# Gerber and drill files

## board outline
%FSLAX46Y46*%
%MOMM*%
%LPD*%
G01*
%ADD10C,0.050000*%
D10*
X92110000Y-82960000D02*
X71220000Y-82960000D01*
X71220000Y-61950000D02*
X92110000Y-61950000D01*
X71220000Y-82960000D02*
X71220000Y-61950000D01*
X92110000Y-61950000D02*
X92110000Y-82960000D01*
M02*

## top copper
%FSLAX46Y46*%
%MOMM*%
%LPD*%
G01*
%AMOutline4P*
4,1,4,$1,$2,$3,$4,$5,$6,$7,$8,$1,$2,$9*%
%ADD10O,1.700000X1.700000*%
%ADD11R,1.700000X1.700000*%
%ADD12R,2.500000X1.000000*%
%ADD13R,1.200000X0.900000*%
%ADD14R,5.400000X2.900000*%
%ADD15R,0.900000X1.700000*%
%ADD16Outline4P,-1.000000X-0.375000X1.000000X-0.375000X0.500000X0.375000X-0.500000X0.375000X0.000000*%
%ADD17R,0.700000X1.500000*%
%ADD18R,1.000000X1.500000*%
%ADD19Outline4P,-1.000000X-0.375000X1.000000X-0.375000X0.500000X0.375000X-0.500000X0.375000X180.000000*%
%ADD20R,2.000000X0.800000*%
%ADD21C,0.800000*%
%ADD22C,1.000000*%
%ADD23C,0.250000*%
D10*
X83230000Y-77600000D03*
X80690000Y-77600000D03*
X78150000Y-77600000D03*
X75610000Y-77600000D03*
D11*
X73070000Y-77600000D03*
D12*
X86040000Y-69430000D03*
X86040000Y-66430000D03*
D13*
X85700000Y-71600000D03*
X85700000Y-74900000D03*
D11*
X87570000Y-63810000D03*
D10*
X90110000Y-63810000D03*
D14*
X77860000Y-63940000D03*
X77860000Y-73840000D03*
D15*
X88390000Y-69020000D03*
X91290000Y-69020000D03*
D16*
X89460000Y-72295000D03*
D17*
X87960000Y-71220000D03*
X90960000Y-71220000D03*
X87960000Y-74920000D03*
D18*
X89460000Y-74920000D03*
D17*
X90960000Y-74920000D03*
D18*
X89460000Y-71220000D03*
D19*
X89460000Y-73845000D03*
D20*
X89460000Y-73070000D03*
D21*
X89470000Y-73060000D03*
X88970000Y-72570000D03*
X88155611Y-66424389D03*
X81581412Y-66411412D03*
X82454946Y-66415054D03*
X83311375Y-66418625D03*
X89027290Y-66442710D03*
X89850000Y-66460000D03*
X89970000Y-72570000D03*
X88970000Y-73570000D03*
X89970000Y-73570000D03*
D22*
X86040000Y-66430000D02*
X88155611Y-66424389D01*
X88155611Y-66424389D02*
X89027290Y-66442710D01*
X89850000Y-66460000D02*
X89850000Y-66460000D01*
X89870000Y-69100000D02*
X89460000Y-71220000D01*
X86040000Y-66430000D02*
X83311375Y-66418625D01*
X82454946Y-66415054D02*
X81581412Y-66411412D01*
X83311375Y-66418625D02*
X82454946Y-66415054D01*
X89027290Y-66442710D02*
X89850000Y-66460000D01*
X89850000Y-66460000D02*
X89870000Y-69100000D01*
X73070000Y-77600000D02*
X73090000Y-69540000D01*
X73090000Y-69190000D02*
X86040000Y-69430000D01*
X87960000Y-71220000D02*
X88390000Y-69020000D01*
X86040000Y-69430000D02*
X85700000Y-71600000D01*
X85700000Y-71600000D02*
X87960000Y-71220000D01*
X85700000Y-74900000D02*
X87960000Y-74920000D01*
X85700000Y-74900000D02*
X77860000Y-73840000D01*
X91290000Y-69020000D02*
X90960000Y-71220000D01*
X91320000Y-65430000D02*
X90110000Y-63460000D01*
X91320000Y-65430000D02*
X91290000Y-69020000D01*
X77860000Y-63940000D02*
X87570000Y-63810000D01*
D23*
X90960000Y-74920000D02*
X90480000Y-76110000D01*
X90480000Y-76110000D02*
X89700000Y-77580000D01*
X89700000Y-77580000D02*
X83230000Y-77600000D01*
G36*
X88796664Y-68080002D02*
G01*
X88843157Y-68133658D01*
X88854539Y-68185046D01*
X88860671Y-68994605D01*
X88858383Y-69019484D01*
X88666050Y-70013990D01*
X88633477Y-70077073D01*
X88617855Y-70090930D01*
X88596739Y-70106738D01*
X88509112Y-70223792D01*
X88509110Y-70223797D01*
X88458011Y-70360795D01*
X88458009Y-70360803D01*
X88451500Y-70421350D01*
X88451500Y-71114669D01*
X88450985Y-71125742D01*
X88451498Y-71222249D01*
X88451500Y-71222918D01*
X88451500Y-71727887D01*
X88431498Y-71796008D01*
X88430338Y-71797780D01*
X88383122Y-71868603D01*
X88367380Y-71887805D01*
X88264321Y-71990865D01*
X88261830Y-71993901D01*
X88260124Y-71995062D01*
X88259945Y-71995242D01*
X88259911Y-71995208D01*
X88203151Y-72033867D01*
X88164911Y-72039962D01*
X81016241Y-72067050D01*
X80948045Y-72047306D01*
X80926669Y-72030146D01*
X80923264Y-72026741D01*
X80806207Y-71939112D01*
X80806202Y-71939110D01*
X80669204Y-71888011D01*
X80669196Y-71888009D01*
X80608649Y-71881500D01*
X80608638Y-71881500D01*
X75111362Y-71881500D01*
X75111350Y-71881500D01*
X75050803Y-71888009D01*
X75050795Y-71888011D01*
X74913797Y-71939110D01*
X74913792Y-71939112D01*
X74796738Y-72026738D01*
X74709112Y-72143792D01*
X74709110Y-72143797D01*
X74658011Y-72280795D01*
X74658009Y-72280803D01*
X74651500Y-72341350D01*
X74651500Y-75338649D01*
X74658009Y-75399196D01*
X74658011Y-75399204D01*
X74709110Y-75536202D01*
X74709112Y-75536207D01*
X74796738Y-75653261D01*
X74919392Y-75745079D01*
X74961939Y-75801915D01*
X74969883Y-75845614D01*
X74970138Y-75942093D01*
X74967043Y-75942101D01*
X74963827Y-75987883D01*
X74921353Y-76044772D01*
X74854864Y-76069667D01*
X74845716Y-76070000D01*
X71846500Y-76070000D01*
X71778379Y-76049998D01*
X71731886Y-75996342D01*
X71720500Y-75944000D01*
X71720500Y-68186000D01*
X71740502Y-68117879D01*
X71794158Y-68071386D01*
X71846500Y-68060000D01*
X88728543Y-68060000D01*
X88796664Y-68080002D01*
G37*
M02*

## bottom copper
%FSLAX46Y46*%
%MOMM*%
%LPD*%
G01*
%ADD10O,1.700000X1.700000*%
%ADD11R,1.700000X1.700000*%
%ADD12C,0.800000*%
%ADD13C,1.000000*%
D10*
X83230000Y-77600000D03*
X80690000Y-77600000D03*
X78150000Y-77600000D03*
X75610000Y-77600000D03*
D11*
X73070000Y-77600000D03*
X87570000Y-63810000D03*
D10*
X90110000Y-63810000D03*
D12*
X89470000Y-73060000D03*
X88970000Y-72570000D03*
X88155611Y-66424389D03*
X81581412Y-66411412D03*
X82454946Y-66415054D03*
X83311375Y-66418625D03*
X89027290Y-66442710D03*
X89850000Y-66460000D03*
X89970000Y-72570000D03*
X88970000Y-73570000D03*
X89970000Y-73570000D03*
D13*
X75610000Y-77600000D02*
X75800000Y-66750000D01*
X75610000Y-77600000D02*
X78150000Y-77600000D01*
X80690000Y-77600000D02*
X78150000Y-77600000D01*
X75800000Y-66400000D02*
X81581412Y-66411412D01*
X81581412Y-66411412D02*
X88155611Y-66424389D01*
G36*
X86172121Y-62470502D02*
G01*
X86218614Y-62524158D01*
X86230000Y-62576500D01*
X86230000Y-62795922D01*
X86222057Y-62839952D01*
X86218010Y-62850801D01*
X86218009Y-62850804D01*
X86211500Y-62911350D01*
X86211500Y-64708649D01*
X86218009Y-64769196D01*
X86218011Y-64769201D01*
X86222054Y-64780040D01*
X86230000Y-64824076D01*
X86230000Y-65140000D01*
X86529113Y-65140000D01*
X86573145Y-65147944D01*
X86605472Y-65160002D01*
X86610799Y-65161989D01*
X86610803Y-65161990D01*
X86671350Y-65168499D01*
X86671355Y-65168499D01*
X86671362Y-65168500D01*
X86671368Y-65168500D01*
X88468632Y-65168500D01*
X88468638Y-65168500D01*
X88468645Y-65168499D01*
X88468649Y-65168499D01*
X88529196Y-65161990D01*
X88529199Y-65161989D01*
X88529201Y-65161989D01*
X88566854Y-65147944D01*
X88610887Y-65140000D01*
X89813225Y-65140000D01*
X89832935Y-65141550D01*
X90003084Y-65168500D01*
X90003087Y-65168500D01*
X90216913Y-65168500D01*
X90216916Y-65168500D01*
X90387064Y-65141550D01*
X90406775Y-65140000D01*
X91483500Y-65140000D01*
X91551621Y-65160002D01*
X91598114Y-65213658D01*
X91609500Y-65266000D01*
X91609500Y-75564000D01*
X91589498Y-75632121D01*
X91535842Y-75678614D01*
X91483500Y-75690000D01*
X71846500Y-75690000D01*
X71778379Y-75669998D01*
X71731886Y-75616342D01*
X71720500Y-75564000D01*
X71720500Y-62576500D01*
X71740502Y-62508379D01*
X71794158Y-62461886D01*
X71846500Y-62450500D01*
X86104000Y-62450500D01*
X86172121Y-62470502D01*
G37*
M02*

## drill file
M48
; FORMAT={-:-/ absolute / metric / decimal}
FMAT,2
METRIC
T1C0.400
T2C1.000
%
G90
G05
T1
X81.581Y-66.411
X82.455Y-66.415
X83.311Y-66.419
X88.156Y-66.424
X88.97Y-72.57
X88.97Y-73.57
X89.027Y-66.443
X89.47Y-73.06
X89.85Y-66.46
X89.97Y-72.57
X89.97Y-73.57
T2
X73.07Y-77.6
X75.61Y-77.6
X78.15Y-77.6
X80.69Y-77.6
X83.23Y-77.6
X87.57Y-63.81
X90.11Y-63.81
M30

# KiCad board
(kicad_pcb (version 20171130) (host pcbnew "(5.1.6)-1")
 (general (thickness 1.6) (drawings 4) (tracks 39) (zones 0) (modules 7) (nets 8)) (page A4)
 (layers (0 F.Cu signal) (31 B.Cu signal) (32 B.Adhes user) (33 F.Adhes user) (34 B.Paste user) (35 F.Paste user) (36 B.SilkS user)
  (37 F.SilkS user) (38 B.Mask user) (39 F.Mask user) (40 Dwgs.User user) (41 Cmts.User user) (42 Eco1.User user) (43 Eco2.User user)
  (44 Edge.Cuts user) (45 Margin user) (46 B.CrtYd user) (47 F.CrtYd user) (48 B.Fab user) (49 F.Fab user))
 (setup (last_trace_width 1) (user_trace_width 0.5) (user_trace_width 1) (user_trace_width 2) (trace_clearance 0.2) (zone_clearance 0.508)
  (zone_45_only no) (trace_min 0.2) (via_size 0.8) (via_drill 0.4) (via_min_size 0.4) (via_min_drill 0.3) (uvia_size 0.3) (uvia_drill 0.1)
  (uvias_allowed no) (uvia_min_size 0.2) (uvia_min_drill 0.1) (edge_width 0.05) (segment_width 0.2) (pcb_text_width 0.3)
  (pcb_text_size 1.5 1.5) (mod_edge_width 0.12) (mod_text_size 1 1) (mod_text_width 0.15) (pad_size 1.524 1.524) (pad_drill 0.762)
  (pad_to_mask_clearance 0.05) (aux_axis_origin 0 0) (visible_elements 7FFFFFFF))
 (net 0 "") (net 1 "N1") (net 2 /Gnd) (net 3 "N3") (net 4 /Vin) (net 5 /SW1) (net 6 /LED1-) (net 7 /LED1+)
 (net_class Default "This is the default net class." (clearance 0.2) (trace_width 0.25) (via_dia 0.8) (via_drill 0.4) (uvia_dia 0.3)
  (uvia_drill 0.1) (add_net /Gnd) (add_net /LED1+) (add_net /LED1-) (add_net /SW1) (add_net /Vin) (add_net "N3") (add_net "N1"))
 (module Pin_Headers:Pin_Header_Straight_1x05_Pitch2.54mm (layer F.Cu) (at 73.07 77.6 90)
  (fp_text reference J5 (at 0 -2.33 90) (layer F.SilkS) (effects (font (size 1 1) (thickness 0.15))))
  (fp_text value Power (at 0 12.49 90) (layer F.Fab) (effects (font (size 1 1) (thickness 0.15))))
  (pad 5 thru_hole oval (at 0 10.16 90) (size 1.7 1.7) (drill 1) (layers *.Cu *.Mask) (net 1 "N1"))
  (pad 4 thru_hole oval (at 0 7.62 90) (size 1.7 1.7) (drill 1) (layers *.Cu *.Mask) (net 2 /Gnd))
  (pad 3 thru_hole oval (at 0 5.08 90) (size 1.7 1.7) (drill 1) (layers *.Cu *.Mask) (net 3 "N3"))
  (pad 2 thru_hole oval (at 0 2.54 90) (size 1.7 1.7) (drill 1) (layers *.Cu *.Mask) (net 2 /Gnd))
  (pad 1 thru_hole rect (at 0 0 90) (size 1.7 1.7) (drill 1) (layers *.Cu *.Mask) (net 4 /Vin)))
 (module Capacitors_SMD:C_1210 (layer F.Cu) (at 86.04 67.93 90)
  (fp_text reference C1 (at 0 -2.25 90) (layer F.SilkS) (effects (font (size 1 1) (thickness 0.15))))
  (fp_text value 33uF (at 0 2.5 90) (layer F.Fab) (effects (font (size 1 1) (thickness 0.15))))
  (pad 1 smd rect (at -1.5 0 90) (size 1 2.5) (layers F.Cu F.Paste F.Mask) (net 4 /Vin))
  (pad 2 smd rect (at 1.5 0 90) (size 1 2.5) (layers F.Cu F.Paste F.Mask) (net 2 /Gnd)))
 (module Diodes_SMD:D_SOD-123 (layer F.Cu) (at 85.7 73.25 270)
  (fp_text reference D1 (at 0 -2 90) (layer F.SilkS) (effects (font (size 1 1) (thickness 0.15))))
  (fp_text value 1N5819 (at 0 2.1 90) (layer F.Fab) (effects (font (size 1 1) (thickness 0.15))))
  (pad 1 smd rect (at -1.65 0 270) (size 0.9 1.2) (layers F.Cu F.Paste F.Mask) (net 4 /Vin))
  (pad 2 smd rect (at 1.65 0 270) (size 0.9 1.2) (layers F.Cu F.Paste F.Mask) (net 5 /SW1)))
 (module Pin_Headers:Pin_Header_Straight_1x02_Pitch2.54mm (layer F.Cu) (at 87.57 63.81 90)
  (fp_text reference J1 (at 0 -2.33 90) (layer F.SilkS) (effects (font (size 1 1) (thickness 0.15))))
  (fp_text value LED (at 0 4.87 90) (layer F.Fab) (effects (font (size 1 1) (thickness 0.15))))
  (pad 1 thru_hole rect (at 0 0 90) (size 1.7 1.7) (drill 1) (layers *.Cu *.Mask) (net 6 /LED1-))
  (pad 2 thru_hole oval (at 0 2.54 90) (size 1.7 1.7) (drill 1) (layers *.Cu *.Mask) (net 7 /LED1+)))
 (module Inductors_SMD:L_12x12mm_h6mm (layer F.Cu) (at 77.86 68.89 270)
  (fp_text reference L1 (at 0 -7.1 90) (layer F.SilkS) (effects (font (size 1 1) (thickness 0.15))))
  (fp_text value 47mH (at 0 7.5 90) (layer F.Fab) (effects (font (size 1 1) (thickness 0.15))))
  (pad 1 smd rect (at -4.95 0 270) (size 2.9 5.4) (layers F.Cu F.Paste F.Mask) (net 6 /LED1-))
  (pad 2 smd rect (at 4.95 0 270) (size 2.9 5.4) (layers F.Cu F.Paste F.Mask) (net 5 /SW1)))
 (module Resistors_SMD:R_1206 (layer F.Cu) (at 89.84 69.02)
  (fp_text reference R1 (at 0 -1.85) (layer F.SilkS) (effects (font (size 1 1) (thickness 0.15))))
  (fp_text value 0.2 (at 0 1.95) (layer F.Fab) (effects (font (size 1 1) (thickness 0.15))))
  (pad 1 smd rect (at -1.45 0) (size 0.9 1.7) (layers F.Cu F.Paste F.Mask) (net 4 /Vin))
  (pad 2 smd rect (at 1.45 0) (size 0.9 1.7) (layers F.Cu F.Paste F.Mask) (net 7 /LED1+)))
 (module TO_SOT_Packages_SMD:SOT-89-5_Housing (layer F.Cu) (at 89.46 73.07 90)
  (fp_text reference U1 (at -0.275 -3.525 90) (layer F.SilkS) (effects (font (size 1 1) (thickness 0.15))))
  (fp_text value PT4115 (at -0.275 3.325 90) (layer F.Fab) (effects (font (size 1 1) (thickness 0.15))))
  (pad 2 smd trapezoid (at 0.775 0) (size 1.5 0.75) (rect_delta 0 0.5) (layers F.Cu F.Paste F.Mask) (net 2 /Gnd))
  (pad 5 smd rect (at 1.85 -1.5) (size 0.7 1.5) (layers F.Cu F.Paste F.Mask) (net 4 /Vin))
  (pad 4 smd rect (at 1.85 1.5) (size 0.7 1.5) (layers F.Cu F.Paste F.Mask) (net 7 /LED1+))
  (pad 1 smd rect (at -1.85 -1.5) (size 0.7 1.5) (layers F.Cu F.Paste F.Mask) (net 5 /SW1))
  (pad 2 smd rect (at -1.85 0) (size 1 1.5) (layers F.Cu F.Paste F.Mask) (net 2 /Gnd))
  (pad 3 smd rect (at -1.85 1.5) (size 0.7 1.5) (layers F.Cu F.Paste F.Mask) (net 1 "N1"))
  (pad 2 smd rect (at 1.85 0) (size 1 1.5) (layers F.Cu F.Paste F.Mask) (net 2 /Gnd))
  (pad 2 smd trapezoid (at -0.775 0 180) (size 1.5 0.75) (rect_delta 0 0.5) (layers F.Cu F.Paste F.Mask) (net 2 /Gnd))
  (pad 2 smd rect (at 0 0) (size 2 0.8) (layers F.Cu F.Paste F.Mask) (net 2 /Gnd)))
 (gr_line (start 92.11 82.96) (end 71.22 82.96) (layer Edge.Cuts) (width 0.05))
 (gr_line (start 71.22 61.95) (end 92.11 61.95) (layer Edge.Cuts) (width 0.05))
 (gr_line (start 71.22 82.96) (end 71.22 61.95) (layer Edge.Cuts) (width 0.05))
 (gr_line (start 92.11 61.95) (end 92.11 82.96) (layer Edge.Cuts) (width 0.05))
 (via (at 89.47 73.06) (size 0.8) (drill 0.4) (layers F.Cu B.Cu) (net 2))
 (via (at 88.97 72.57) (size 0.8) (drill 0.4) (layers F.Cu B.Cu) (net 2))
 (segment (start 75.61 77.6) (end 75.8 66.75) (width 1) (layer B.Cu) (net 2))
 (via (at 88.155611 66.424389) (size 0.8) (drill 0.4) (layers F.Cu B.Cu) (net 2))
 (segment (start 75.61 77.6) (end 78.15 77.6) (width 1) (layer B.Cu) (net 2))
 (segment (start 86.04 66.43) (end 88.155611 66.424389) (width 1) (layer F.Cu) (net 2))
 (segment (start 88.155611 66.424389) (end 89.02729 66.44271) (width 1) (layer F.Cu) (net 2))
 (segment (start 89.85 66.46) (end 89.85 66.46) (width 1) (layer F.Cu) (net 2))
 (segment (start 89.87 69.1) (end 89.46 71.22) (width 1) (layer F.Cu) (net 2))
 (segment (start 80.69 77.6) (end 78.15 77.6) (width 1) (layer B.Cu) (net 2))
 (via (at 81.581412 66.411412) (size 0.8) (drill 0.4) (layers F.Cu B.Cu) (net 2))
 (segment (start 86.04 66.43) (end 83.311375 66.418625) (width 1) (layer F.Cu) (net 2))
 (segment (start 75.8 66.4) (end 81.581412 66.411412) (width 1) (layer B.Cu) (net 2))
 (segment (start 81.581412 66.411412) (end 88.155611 66.424389) (width 1) (layer B.Cu) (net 2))
 (segment (start 82.454946 66.415054) (end 81.581412 66.411412) (width 1) (layer F.Cu) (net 2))
 (via (at 82.454946 66.415054) (size 0.8) (drill 0.4) (layers F.Cu B.Cu) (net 2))
 (segment (start 83.311375 66.418625) (end 82.454946 66.415054) (width 1) (layer F.Cu) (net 2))
 (via (at 83.311375 66.418625) (size 0.8) (drill 0.4) (layers F.Cu B.Cu) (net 2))
 (segment (start 89.02729 66.44271) (end 89.85 66.46) (width 1) (layer F.Cu) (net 2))
 (via (at 89.02729 66.44271) (size 0.8) (drill 0.4) (layers F.Cu B.Cu) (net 2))
 (segment (start 89.85 66.46) (end 89.87 69.1) (width 1) (layer F.Cu) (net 2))
 (via (at 89.85 66.46) (size 0.8) (drill 0.4) (layers F.Cu B.Cu) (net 2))
 (via (at 89.97 72.57) (size 0.8) (drill 0.4) (layers F.Cu B.Cu) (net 2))
 (via (at 88.97 73.57) (size 0.8) (drill 0.4) (layers F.Cu B.Cu) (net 2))
 (via (at 89.97 73.57) (size 0.8) (drill 0.4) (layers F.Cu B.Cu) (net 2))
 (segment (start 73.07 77.6) (end 73.09 69.54) (width 1) (layer F.Cu) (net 4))
 (segment (start 73.09 69.19) (end 86.04 69.43) (width 1) (layer F.Cu) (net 4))
 (segment (start 87.96 71.22) (end 88.39 69.02) (width 1) (layer F.Cu) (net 4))
 (segment (start 86.04 69.43) (end 85.7 71.6) (width 1) (layer F.Cu) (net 4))
 (segment (start 85.7 71.6) (end 87.96 71.22) (width 1) (layer F.Cu) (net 4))
 (segment (start 85.7 74.9) (end 87.96 74.92) (width 1) (layer F.Cu) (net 5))
 (segment (start 85.7 74.9) (end 77.86 73.84) (width 1) (layer F.Cu) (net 5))
 (segment (start 91.29 69.02) (end 90.96 71.22) (width 1) (layer F.Cu) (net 7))
 (segment (start 91.32 65.43) (end 90.11 63.46) (width 1) (layer F.Cu) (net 7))
 (segment (start 91.32 65.43) (end 91.29 69.02) (width 1) (layer F.Cu) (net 7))
 (segment (start 77.86 63.94) (end 87.57 63.81) (width 1) (layer F.Cu) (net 6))
 (segment (start 90.96 74.92) (end 90.48 76.11) (width 0.25) (layer F.Cu) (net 1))
 (segment (start 90.48 76.11) (end 89.7 77.58) (width 0.25) (layer F.Cu) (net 1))
 (segment (start 89.7 77.58) (end 83.23 77.6) (width 0.25) (layer F.Cu) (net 1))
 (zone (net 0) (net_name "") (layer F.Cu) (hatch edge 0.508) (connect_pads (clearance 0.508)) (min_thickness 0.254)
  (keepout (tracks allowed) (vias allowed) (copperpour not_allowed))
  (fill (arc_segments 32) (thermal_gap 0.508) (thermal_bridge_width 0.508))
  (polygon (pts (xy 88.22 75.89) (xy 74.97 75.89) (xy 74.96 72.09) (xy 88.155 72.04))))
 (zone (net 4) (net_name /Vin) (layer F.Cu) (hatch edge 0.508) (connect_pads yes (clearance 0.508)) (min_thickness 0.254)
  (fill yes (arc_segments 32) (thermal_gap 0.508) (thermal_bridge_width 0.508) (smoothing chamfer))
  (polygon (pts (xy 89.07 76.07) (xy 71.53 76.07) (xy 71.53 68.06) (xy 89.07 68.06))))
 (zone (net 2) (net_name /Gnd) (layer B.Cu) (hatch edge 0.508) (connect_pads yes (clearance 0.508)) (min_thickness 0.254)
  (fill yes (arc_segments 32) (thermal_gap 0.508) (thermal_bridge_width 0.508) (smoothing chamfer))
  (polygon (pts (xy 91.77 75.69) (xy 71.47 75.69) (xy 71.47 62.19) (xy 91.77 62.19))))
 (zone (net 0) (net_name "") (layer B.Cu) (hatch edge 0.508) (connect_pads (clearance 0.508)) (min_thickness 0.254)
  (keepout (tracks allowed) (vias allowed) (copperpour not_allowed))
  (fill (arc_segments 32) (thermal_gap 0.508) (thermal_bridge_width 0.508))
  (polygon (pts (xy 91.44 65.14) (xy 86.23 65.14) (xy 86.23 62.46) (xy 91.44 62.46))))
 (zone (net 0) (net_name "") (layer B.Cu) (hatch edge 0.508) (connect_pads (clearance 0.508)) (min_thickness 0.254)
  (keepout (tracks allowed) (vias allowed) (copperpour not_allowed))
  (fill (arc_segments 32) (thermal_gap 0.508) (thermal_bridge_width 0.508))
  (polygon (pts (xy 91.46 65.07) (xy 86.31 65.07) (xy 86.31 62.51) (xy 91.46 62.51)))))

